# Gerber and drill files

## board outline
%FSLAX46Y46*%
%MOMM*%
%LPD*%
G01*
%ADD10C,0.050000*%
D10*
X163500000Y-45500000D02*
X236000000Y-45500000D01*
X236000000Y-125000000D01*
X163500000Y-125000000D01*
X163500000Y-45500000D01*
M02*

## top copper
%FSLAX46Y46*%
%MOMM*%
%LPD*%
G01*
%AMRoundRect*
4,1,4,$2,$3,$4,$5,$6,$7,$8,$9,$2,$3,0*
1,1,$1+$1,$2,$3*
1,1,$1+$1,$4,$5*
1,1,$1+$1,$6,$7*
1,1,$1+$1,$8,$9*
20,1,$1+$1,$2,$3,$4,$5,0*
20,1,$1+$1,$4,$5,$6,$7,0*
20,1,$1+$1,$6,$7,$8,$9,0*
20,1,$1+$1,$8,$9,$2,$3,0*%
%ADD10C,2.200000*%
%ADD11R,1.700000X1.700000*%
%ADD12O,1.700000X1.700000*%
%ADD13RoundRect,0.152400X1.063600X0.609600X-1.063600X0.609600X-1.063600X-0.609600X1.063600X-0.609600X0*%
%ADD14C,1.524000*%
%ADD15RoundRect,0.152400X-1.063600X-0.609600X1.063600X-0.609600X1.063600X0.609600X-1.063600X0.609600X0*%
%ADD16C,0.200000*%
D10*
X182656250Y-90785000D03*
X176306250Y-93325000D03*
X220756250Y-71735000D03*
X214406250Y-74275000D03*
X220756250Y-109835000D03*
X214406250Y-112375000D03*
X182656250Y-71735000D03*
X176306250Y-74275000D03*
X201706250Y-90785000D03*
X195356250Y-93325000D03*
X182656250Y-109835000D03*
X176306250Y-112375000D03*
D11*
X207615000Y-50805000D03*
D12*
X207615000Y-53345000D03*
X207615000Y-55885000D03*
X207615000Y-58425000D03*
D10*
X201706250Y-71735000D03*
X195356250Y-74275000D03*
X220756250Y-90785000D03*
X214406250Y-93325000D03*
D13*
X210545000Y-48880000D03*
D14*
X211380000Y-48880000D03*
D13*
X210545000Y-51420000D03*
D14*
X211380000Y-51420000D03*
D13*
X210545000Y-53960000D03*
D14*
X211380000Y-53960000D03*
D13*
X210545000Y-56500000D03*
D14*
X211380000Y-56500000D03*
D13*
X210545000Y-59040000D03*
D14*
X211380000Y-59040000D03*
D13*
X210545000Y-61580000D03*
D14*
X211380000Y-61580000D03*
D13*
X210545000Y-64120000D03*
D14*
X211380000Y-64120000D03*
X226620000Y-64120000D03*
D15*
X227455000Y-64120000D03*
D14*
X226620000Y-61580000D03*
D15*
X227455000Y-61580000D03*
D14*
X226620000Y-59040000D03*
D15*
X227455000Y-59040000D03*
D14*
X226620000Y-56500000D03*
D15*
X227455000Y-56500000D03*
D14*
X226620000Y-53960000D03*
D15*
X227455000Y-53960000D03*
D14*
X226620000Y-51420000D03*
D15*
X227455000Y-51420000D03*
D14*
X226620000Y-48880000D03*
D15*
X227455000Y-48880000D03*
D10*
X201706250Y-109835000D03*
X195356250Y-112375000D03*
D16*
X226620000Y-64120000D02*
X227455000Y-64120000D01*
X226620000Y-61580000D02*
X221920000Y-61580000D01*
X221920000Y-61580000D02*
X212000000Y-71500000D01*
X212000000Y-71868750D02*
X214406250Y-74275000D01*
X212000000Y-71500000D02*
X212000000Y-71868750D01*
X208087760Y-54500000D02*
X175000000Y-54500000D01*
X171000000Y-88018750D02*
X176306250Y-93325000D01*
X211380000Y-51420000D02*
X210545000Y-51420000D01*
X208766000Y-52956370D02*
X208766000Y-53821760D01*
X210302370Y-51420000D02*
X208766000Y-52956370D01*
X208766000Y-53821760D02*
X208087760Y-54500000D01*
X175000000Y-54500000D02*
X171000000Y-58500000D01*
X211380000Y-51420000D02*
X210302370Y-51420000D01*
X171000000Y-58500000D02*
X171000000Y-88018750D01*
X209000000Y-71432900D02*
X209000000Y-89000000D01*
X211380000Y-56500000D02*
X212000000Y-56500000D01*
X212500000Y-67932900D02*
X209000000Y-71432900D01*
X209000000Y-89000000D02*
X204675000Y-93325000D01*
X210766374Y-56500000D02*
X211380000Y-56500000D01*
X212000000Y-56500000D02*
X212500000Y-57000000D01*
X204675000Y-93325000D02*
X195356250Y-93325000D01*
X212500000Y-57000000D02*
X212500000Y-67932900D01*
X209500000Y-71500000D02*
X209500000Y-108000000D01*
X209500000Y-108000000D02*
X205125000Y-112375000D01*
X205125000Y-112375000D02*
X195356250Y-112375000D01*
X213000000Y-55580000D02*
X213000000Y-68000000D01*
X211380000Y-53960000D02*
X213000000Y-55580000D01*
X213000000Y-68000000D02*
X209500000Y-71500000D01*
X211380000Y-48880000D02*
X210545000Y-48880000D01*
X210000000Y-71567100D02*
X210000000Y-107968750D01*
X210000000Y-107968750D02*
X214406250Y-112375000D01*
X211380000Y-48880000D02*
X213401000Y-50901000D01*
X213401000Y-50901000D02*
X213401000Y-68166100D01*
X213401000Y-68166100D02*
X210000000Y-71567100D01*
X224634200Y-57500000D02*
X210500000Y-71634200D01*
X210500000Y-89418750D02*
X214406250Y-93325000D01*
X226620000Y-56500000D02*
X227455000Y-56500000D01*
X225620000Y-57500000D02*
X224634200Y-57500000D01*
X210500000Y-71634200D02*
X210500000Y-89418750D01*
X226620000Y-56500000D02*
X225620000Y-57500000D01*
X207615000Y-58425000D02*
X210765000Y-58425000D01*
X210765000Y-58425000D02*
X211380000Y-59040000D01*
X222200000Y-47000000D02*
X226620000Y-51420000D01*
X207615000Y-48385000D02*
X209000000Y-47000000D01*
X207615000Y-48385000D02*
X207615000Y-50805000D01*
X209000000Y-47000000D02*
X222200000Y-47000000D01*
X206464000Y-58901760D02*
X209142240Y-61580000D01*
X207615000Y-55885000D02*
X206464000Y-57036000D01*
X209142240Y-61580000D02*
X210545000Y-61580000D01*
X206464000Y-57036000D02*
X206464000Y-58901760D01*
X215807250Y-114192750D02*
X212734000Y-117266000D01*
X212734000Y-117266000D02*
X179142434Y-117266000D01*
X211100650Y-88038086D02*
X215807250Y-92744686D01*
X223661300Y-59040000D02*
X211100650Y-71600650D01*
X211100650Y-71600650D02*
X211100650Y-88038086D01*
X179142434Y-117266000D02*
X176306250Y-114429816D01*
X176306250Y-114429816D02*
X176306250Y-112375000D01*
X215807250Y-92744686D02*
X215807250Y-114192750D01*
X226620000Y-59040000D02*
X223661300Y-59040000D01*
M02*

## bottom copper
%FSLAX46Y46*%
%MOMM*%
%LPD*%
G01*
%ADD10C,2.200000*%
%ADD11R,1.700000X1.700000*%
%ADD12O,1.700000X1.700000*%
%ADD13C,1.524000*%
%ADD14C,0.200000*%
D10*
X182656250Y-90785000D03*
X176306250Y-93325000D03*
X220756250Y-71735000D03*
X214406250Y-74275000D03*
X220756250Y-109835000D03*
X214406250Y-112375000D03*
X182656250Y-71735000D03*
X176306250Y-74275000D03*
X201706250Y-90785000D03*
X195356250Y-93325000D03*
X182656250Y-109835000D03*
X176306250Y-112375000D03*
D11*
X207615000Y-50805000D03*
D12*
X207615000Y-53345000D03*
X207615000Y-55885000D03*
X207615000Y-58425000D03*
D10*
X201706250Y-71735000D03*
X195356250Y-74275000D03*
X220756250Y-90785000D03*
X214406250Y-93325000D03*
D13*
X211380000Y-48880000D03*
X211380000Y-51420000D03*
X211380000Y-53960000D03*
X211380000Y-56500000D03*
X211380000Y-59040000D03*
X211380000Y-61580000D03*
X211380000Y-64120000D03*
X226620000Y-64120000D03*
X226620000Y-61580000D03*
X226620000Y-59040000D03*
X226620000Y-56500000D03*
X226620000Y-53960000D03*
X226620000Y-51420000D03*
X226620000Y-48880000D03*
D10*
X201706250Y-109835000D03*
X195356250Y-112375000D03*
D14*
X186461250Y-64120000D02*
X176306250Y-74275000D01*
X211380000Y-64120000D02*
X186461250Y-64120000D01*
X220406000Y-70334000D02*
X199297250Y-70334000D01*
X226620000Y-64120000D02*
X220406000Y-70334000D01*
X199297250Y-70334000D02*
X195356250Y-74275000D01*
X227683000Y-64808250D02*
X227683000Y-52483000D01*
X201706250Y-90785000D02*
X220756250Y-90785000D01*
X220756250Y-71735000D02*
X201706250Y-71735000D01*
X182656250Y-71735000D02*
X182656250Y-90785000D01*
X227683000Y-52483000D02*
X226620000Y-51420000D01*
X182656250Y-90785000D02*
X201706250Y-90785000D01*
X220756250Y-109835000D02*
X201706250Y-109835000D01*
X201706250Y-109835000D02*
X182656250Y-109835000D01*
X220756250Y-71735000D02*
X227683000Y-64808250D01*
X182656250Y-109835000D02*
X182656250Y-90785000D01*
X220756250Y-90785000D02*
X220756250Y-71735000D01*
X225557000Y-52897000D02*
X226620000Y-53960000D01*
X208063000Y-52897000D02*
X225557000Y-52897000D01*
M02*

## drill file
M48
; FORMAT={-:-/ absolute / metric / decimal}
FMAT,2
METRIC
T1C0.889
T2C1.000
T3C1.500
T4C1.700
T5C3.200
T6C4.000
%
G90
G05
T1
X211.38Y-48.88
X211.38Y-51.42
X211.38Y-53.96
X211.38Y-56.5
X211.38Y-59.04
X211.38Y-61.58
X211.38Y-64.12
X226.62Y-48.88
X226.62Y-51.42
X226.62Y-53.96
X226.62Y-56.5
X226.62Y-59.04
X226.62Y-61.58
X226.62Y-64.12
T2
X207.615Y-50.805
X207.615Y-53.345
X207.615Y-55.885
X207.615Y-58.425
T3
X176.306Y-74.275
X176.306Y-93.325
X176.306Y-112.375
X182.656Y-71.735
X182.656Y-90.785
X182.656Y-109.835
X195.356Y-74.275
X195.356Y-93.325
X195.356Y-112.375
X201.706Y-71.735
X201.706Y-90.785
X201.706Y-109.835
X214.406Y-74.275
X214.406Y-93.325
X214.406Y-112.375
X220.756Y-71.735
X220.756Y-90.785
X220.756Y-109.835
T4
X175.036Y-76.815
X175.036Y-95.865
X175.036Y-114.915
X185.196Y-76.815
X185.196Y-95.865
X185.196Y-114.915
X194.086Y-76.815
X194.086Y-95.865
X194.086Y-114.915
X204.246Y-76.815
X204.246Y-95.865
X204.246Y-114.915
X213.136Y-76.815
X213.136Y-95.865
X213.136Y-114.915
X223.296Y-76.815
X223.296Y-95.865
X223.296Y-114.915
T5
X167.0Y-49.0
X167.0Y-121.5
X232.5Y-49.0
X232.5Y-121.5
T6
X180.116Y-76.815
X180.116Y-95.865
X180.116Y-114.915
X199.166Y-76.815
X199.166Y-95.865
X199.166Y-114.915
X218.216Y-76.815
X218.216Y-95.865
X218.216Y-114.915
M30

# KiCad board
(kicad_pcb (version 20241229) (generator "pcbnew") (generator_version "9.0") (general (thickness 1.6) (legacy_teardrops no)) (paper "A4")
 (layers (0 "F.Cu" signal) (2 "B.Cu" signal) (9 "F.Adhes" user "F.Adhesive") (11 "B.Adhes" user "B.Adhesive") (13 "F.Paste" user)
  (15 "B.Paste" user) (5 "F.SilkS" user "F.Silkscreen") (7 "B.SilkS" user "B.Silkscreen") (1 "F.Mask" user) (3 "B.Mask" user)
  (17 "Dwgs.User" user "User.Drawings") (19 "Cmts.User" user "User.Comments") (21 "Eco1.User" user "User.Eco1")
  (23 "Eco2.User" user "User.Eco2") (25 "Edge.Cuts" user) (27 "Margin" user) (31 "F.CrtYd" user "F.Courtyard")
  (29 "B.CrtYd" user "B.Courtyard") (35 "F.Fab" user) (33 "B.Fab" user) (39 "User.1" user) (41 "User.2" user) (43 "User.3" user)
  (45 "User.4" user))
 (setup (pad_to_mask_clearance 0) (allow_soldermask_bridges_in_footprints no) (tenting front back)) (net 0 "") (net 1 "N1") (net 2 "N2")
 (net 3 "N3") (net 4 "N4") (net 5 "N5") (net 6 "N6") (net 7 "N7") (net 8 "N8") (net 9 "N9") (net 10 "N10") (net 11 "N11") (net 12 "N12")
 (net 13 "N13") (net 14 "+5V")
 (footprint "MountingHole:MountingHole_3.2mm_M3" (layer "F.Cu") (at 232.5 49)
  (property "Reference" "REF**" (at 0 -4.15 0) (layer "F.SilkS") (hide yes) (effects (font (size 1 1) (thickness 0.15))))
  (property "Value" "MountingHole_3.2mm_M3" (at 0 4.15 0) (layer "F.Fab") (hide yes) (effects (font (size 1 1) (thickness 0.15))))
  (pad "" np_thru_hole circle (at 0 0) (size 3.2 3.2) (drill 3.2) (layers "*.Cu" "*.Mask")))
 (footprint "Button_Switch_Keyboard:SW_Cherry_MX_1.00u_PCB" (layer "F.Cu") (at 182.65625 90.785)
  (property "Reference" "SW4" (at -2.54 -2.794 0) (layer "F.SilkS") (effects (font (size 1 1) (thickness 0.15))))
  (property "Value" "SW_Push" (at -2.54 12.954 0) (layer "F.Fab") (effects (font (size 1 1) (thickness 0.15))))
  (pad "" np_thru_hole circle (at -7.62 5.08) (size 1.7 1.7) (drill 1.7) (layers "*.Cu" "*.Mask"))
  (pad "" np_thru_hole circle (at -2.54 5.08) (size 4 4) (drill 4) (layers "*.Cu" "*.Mask"))
  (pad "" np_thru_hole circle (at 2.54 5.08) (size 1.7 1.7) (drill 1.7) (layers "*.Cu" "*.Mask"))
  (pad "1" thru_hole circle (at 0 0) (size 2.2 2.2) (drill 1.5) (layers "*.Cu" "*.Mask") (remove_unused_layers no) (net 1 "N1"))
  (pad "2" thru_hole circle (at -6.35 2.54) (size 2.2 2.2) (drill 1.5) (layers "*.Cu" "*.Mask") (remove_unused_layers no) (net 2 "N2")))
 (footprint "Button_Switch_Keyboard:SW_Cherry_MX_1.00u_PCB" (layer "F.Cu") (at 220.75625 71.735)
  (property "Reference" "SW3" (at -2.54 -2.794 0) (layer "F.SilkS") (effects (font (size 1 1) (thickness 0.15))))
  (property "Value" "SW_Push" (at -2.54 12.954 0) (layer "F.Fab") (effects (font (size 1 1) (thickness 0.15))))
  (pad "" np_thru_hole circle (at -7.62 5.08) (size 1.7 1.7) (drill 1.7) (layers "*.Cu" "*.Mask"))
  (pad "" np_thru_hole circle (at -2.54 5.08) (size 4 4) (drill 4) (layers "*.Cu" "*.Mask"))
  (pad "" np_thru_hole circle (at 2.54 5.08) (size 1.7 1.7) (drill 1.7) (layers "*.Cu" "*.Mask"))
  (pad "1" thru_hole circle (at 0 0) (size 2.2 2.2) (drill 1.5) (layers "*.Cu" "*.Mask") (remove_unused_layers no) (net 1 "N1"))
  (pad "2" thru_hole circle (at -6.35 2.54) (size 2.2 2.2) (drill 1.5) (layers "*.Cu" "*.Mask") (remove_unused_layers no) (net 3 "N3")))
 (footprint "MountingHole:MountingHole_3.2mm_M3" (layer "F.Cu") (at 167 121.5)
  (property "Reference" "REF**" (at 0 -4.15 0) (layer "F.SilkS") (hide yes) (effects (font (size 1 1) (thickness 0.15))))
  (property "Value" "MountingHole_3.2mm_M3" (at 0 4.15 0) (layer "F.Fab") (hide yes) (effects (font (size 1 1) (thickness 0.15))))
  (pad "" np_thru_hole circle (at 0 0) (size 3.2 3.2) (drill 3.2) (layers "*.Cu" "*.Mask")))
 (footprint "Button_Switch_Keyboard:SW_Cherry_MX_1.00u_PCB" (layer "F.Cu") (at 220.75625 109.835)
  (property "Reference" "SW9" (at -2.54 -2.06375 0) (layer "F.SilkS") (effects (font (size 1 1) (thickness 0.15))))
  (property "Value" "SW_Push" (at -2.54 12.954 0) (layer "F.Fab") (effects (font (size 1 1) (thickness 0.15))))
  (pad "" np_thru_hole circle (at -7.62 5.08) (size 1.7 1.7) (drill 1.7) (layers "*.Cu" "*.Mask"))
  (pad "" np_thru_hole circle (at -2.54 5.08) (size 4 4) (drill 4) (layers "*.Cu" "*.Mask"))
  (pad "" np_thru_hole circle (at 2.54 5.08) (size 1.7 1.7) (drill 1.7) (layers "*.Cu" "*.Mask"))
  (pad "1" thru_hole circle (at 0 0) (size 2.2 2.2) (drill 1.5) (layers "*.Cu" "*.Mask") (remove_unused_layers no) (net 1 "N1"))
  (pad "2" thru_hole circle (at -6.35 2.54) (size 2.2 2.2) (drill 1.5) (layers "*.Cu" "*.Mask") (remove_unused_layers no) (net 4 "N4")))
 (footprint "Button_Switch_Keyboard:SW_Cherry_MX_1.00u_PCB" (layer "F.Cu") (at 182.65625 71.735)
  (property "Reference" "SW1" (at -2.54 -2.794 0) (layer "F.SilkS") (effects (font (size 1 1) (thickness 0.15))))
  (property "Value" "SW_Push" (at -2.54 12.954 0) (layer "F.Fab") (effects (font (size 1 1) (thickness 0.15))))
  (pad "" np_thru_hole circle (at -7.62 5.08) (size 1.7 1.7) (drill 1.7) (layers "*.Cu" "*.Mask"))
  (pad "" np_thru_hole circle (at -2.54 5.08) (size 4 4) (drill 4) (layers "*.Cu" "*.Mask"))
  (pad "" np_thru_hole circle (at 2.54 5.08) (size 1.7 1.7) (drill 1.7) (layers "*.Cu" "*.Mask"))
  (pad "1" thru_hole circle (at 0 0) (size 2.2 2.2) (drill 1.5) (layers "*.Cu" "*.Mask") (remove_unused_layers no) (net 1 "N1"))
  (pad "2" thru_hole circle (at -6.35 2.54) (size 2.2 2.2) (drill 1.5) (layers "*.Cu" "*.Mask") (remove_unused_layers no) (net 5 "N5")))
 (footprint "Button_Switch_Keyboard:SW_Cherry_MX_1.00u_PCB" (layer "F.Cu") (at 201.70625 90.785)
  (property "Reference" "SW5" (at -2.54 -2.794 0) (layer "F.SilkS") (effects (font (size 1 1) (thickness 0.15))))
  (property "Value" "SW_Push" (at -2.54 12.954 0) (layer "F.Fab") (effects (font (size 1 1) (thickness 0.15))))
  (pad "" np_thru_hole circle (at -7.62 5.08) (size 1.7 1.7) (drill 1.7) (layers "*.Cu" "*.Mask"))
  (pad "" np_thru_hole circle (at -2.54 5.08) (size 4 4) (drill 4) (layers "*.Cu" "*.Mask"))
  (pad "" np_thru_hole circle (at 2.54 5.08) (size 1.7 1.7) (drill 1.7) (layers "*.Cu" "*.Mask"))
  (pad "1" thru_hole circle (at 0 0) (size 2.2 2.2) (drill 1.5) (layers "*.Cu" "*.Mask") (remove_unused_layers no) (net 1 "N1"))
  (pad "2" thru_hole circle (at -6.35 2.54) (size 2.2 2.2) (drill 1.5) (layers "*.Cu" "*.Mask") (remove_unused_layers no) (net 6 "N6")))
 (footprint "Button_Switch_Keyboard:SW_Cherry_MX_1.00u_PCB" (layer "F.Cu") (at 182.65625 109.835)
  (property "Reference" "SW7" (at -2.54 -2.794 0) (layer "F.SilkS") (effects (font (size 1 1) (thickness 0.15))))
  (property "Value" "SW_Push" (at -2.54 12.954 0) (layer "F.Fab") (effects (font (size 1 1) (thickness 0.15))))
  (pad "" np_thru_hole circle (at -7.62 5.08) (size 1.7 1.7) (drill 1.7) (layers "*.Cu" "*.Mask"))
  (pad "" np_thru_hole circle (at -2.54 5.08) (size 4 4) (drill 4) (layers "*.Cu" "*.Mask"))
  (pad "" np_thru_hole circle (at 2.54 5.08) (size 1.7 1.7) (drill 1.7) (layers "*.Cu" "*.Mask"))
  (pad "1" thru_hole circle (at 0 0) (size 2.2 2.2) (drill 1.5) (layers "*.Cu" "*.Mask") (remove_unused_layers no) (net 1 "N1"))
  (pad "2" thru_hole circle (at -6.35 2.54) (size 2.2 2.2) (drill 1.5) (layers "*.Cu" "*.Mask") (remove_unused_layers no) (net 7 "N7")))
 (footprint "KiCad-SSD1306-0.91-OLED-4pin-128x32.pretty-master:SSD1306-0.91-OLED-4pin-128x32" (layer "F.Cu") (at 171.115 48.615)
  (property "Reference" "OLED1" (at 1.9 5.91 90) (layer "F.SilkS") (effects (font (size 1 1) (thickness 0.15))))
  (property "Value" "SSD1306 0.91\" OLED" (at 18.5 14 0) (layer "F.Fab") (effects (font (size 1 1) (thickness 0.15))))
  (pad "1" thru_hole rect (at 36.5 2.19) (size 1.7 1.7) (drill 1) (layers "*.Cu" "*.Mask") (remove_unused_layers no) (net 1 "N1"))
  (pad "2" thru_hole oval (at 36.5 4.73) (size 1.7 1.7) (drill 1) (layers "*.Cu" "*.Mask") (remove_unused_layers no) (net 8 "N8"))
  (pad "3" thru_hole oval (at 36.5 7.27) (size 1.7 1.7) (drill 1) (layers "*.Cu" "*.Mask") (remove_unused_layers no) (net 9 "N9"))
  (pad "4" thru_hole oval (at 36.5 9.81) (size 1.7 1.7) (drill 1) (layers "*.Cu" "*.Mask") (remove_unused_layers no) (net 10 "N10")))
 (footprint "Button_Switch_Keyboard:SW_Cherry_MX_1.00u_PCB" (layer "F.Cu") (at 201.70625 71.735)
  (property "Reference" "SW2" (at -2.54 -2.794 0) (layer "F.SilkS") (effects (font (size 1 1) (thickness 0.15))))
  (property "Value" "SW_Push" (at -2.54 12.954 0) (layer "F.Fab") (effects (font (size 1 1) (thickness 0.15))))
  (pad "" np_thru_hole circle (at -7.62 5.08) (size 1.7 1.7) (drill 1.7) (layers "*.Cu" "*.Mask"))
  (pad "" np_thru_hole circle (at -2.54 5.08) (size 4 4) (drill 4) (layers "*.Cu" "*.Mask"))
  (pad "" np_thru_hole circle (at 2.54 5.08) (size 1.7 1.7) (drill 1.7) (layers "*.Cu" "*.Mask"))
  (pad "1" thru_hole circle (at 0 0) (size 2.2 2.2) (drill 1.5) (layers "*.Cu" "*.Mask") (remove_unused_layers no) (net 1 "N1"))
  (pad "2" thru_hole circle (at -6.35 2.54) (size 2.2 2.2) (drill 1.5) (layers "*.Cu" "*.Mask") (remove_unused_layers no) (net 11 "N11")))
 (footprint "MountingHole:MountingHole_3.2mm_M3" (layer "F.Cu") (at 167 49)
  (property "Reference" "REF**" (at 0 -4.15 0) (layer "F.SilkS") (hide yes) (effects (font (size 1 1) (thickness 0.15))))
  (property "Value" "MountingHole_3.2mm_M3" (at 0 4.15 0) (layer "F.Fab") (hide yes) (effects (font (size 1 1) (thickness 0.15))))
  (pad "" np_thru_hole circle (at 0 0) (size 3.2 3.2) (drill 3.2) (layers "*.Cu" "*.Mask")))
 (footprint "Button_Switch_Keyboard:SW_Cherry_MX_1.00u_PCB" (layer "F.Cu") (at 220.75625 90.785)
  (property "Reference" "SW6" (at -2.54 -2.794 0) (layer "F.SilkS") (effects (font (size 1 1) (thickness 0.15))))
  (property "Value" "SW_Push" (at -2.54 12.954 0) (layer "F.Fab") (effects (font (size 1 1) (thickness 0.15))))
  (pad "" np_thru_hole circle (at -7.62 5.08) (size 1.7 1.7) (drill 1.7) (layers "*.Cu" "*.Mask"))
  (pad "" np_thru_hole circle (at -2.54 5.08) (size 4 4) (drill 4) (layers "*.Cu" "*.Mask"))
  (pad "" np_thru_hole circle (at 2.54 5.08) (size 1.7 1.7) (drill 1.7) (layers "*.Cu" "*.Mask"))
  (pad "1" thru_hole circle (at 0 0) (size 2.2 2.2) (drill 1.5) (layers "*.Cu" "*.Mask") (remove_unused_layers no) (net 1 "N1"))
  (pad "2" thru_hole circle (at -6.35 2.54) (size 2.2 2.2) (drill 1.5) (layers "*.Cu" "*.Mask") (remove_unused_layers no) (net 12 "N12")))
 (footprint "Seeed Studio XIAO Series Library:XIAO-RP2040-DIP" (layer "F.Cu") (at 219 56.5)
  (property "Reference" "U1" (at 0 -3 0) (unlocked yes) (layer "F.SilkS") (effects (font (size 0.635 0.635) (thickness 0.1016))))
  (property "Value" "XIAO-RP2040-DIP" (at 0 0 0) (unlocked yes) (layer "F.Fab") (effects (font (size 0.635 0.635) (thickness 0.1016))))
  (pad "1" smd roundrect (at -8.455 -7.62 180) (size 2.432 1.524) (layers "F.Cu" "F.Mask") (roundrect_rratio 0.1) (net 4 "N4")
   (thermal_bridge_angle 45))
  (pad "1" thru_hole circle (at -7.62 -7.62 180) (size 1.524 1.524) (drill 0.889) (layers "*.Cu" "*.Mask") (remove_unused_layers no)
   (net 4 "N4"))
  (pad "2" smd roundrect (at -8.455 -5.08 180) (size 2.432 1.524) (layers "F.Cu" "F.Mask") (roundrect_rratio 0.1) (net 2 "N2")
   (thermal_bridge_angle 45))
  (pad "2" thru_hole circle (at -7.62 -5.08 180) (size 1.524 1.524) (drill 0.889) (layers "*.Cu" "*.Mask") (remove_unused_layers no)
   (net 2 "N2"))
  (pad "3" smd roundrect (at -8.455 -2.54 180) (size 2.432 1.524) (layers "F.Cu" "F.Mask") (roundrect_rratio 0.1) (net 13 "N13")
   (thermal_bridge_angle 45))
  (pad "3" thru_hole circle (at -7.62 -2.54 180) (size 1.524 1.524) (drill 0.889) (layers "*.Cu" "*.Mask") (remove_unused_layers no)
   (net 13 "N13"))
  (pad "4" smd roundrect (at -8.455 0 180) (size 2.432 1.524) (layers "F.Cu" "F.Mask") (roundrect_rratio 0.1) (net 6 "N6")
   (thermal_bridge_angle 45))
  (pad "4" thru_hole circle (at -7.62 0 180) (size 1.524 1.524) (drill 0.889) (layers "*.Cu" "*.Mask") (remove_unused_layers no)
   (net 6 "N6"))
  (pad "5" smd roundrect (at -8.455 2.54 180) (size 2.432 1.524) (layers "F.Cu" "F.Mask") (roundrect_rratio 0.1) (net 10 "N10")
   (thermal_bridge_angle 45))
  (pad "5" thru_hole circle (at -7.62 2.54 180) (size 1.524 1.524) (drill 0.889) (layers "*.Cu" "*.Mask") (remove_unused_layers no)
   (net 10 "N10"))
  (pad "6" smd roundrect (at -8.455 5.08 180) (size 2.432 1.524) (layers "F.Cu" "F.Mask") (roundrect_rratio 0.1) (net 9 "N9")
   (thermal_bridge_angle 45))
  (pad "6" thru_hole circle (at -7.62 5.08 180) (size 1.524 1.524) (drill 0.889) (layers "*.Cu" "*.Mask") (remove_unused_layers no)
   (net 9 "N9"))
  (pad "7" smd roundrect (at -8.455 7.62 180) (size 2.432 1.524) (layers "F.Cu" "F.Mask") (roundrect_rratio 0.1) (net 5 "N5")
   (thermal_bridge_angle 45))
  (pad "7" thru_hole circle (at -7.62 7.62 180) (size 1.524 1.524) (drill 0.889) (layers "*.Cu" "*.Mask") (remove_unused_layers no)
   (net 5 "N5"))
  (pad "8" thru_hole circle (at 7.62 7.62) (size 1.524 1.524) (drill 0.889) (layers "*.Cu" "*.Mask") (remove_unused_layers no)
   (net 11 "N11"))
  (pad "8" smd roundrect (at 8.455 7.62) (size 2.432 1.524) (layers "F.Cu" "F.Mask") (roundrect_rratio 0.1) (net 11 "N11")
   (thermal_bridge_angle 45))
  (pad "9" thru_hole circle (at 7.62 5.08) (size 1.524 1.524) (drill 0.889) (layers "*.Cu" "*.Mask") (remove_unused_layers no) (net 3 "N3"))
  (pad "9" smd roundrect (at 8.455 5.08) (size 2.432 1.524) (layers "F.Cu" "F.Mask") (roundrect_rratio 0.1) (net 3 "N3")
   (thermal_bridge_angle 45))
  (pad "10" thru_hole circle (at 7.62 2.54) (size 1.524 1.524) (drill 0.889) (layers "*.Cu" "*.Mask") (remove_unused_layers no) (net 7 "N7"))
  (pad "10" smd roundrect (at 8.455 2.54) (size 2.432 1.524) (layers "F.Cu" "F.Mask") (roundrect_rratio 0.1) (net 7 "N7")
   (thermal_bridge_angle 45))
  (pad "11" thru_hole circle (at 7.62 0) (size 1.524 1.524) (drill 0.889) (layers "*.Cu" "*.Mask") (remove_unused_layers no) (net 12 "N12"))
  (pad "11" smd roundrect (at 8.455 0) (size 2.432 1.524) (layers "F.Cu" "F.Mask") (roundrect_rratio 0.1) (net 12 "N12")
   (thermal_bridge_angle 45))
  (pad "12" thru_hole circle (at 7.62 -2.54) (size 1.524 1.524) (drill 0.889) (layers "*.Cu" "*.Mask") (remove_unused_layers no)
   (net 8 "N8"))
  (pad "12" smd roundrect (at 8.455 -2.54) (size 2.432 1.524) (layers "F.Cu" "F.Mask") (roundrect_rratio 0.1) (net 8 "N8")
   (thermal_bridge_angle 45))
  (pad "13" thru_hole circle (at 7.62 -5.08) (size 1.524 1.524) (drill 0.889) (layers "*.Cu" "*.Mask") (remove_unused_layers no)
   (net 1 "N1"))
  (pad "13" smd roundrect (at 8.455 -5.08) (size 2.432 1.524) (layers "F.Cu" "F.Mask") (roundrect_rratio 0.1) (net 1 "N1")
   (thermal_bridge_angle 45))
  (pad "14" thru_hole circle (at 7.62 -7.62) (size 1.524 1.524) (drill 0.889) (layers "*.Cu" "*.Mask") (remove_unused_layers no)
   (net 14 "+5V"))
  (pad "14" smd roundrect (at 8.455 -7.62) (size 2.432 1.524) (layers "F.Cu" "F.Mask") (roundrect_rratio 0.1) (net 14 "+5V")
   (thermal_bridge_angle 45)))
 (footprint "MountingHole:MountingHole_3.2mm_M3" (layer "F.Cu") (at 232.5 121.5)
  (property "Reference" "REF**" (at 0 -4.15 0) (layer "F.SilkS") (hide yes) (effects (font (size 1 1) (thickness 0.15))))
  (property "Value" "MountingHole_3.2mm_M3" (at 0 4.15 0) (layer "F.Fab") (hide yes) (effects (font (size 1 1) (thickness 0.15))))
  (pad "" np_thru_hole circle (at 0 0) (size 3.2 3.2) (drill 3.2) (layers "*.Cu" "*.Mask")))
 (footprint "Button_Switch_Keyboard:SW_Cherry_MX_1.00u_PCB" (layer "F.Cu") (at 201.70625 109.835)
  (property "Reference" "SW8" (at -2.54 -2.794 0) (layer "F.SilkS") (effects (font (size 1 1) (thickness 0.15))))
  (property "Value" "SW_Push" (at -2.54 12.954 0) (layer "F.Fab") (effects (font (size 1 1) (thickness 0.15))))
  (pad "" np_thru_hole circle (at -7.62 5.08) (size 1.7 1.7) (drill 1.7) (layers "*.Cu" "*.Mask"))
  (pad "" np_thru_hole circle (at -2.54 5.08) (size 4 4) (drill 4) (layers "*.Cu" "*.Mask"))
  (pad "" np_thru_hole circle (at 2.54 5.08) (size 1.7 1.7) (drill 1.7) (layers "*.Cu" "*.Mask"))
  (pad "1" thru_hole circle (at 0 0) (size 2.2 2.2) (drill 1.5) (layers "*.Cu" "*.Mask") (remove_unused_layers no) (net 1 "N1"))
  (pad "2" thru_hole circle (at -6.35 2.54) (size 2.2 2.2) (drill 1.5) (layers "*.Cu" "*.Mask") (remove_unused_layers no) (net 13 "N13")))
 (gr_rect (start 163.5 45.5) (end 236 125) (stroke (width 0.05) (type default)) (fill no) (layer "Edge.Cuts"))
 (segment (start 186.46125 64.12) (end 176.30625 74.275) (width 0.2) (layer "B.Cu") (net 5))
 (segment (start 211.38 64.12) (end 186.46125 64.12) (width 0.2) (layer "B.Cu") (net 5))
 (segment (start 226.62 64.12) (end 227.455 64.12) (width 0.2) (layer "F.Cu") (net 11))
 (segment (start 220.406 70.334) (end 199.29725 70.334) (width 0.2) (layer "B.Cu") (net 11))
 (segment (start 226.62 64.12) (end 220.406 70.334) (width 0.2) (layer "B.Cu") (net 11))
 (segment (start 199.29725 70.334) (end 195.35625 74.275) (width 0.2) (layer "B.Cu") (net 11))
 (segment (start 226.62 61.58) (end 221.92 61.58) (width 0.2) (layer "F.Cu") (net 3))
 (segment (start 221.92 61.58) (end 212 71.5) (width 0.2) (layer "F.Cu") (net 3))
 (segment (start 212 71.86875) (end 214.40625 74.275) (width 0.2) (layer "F.Cu") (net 3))
 (segment (start 212 71.5) (end 212 71.86875) (width 0.2) (layer "F.Cu") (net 3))
 (segment (start 208.08776 54.5) (end 175 54.5) (width 0.2) (layer "F.Cu") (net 2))
 (segment (start 171 88.01875) (end 176.30625 93.325) (width 0.2) (layer "F.Cu") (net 2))
 (segment (start 211.38 51.42) (end 210.545 51.42) (width 0.2) (layer "F.Cu") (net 2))
 (segment (start 208.766 52.95637) (end 208.766 53.82176) (width 0.2) (layer "F.Cu") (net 2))
 (segment (start 210.30237 51.42) (end 208.766 52.95637) (width 0.2) (layer "F.Cu") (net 2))
 (segment (start 208.766 53.82176) (end 208.08776 54.5) (width 0.2) (layer "F.Cu") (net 2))
 (segment (start 175 54.5) (end 171 58.5) (width 0.2) (layer "F.Cu") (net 2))
 (segment (start 211.38 51.42) (end 210.30237 51.42) (width 0.2) (layer "F.Cu") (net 2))
 (segment (start 171 58.5) (end 171 88.01875) (width 0.2) (layer "F.Cu") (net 2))
 (segment (start 209 71.4329) (end 209 89) (width 0.2) (layer "F.Cu") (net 6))
 (segment (start 211.38 56.5) (end 212 56.5) (width 0.2) (layer "F.Cu") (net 6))
 (segment (start 212.5 67.9329) (end 209 71.4329) (width 0.2) (layer "F.Cu") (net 6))
 (segment (start 209 89) (end 204.675 93.325) (width 0.2) (layer "F.Cu") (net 6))
 (segment (start 210.766374 56.5) (end 211.38 56.5) (width 0.2) (layer "F.Cu") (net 6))
 (segment (start 212 56.5) (end 212.5 57) (width 0.2) (layer "F.Cu") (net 6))
 (segment (start 204.675 93.325) (end 195.35625 93.325) (width 0.2) (layer "F.Cu") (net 6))
 (segment (start 212.5 57) (end 212.5 67.9329) (width 0.2) (layer "F.Cu") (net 6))
 (segment (start 209.5 71.5) (end 209.5 108) (width 0.2) (layer "F.Cu") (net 13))
 (segment (start 209.5 108) (end 205.125 112.375) (width 0.2) (layer "F.Cu") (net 13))
 (segment (start 205.125 112.375) (end 195.35625 112.375) (width 0.2) (layer "F.Cu") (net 13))
 (segment (start 213 55.58) (end 213 68) (width 0.2) (layer "F.Cu") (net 13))
 (segment (start 211.38 53.96) (end 213 55.58) (width 0.2) (layer "F.Cu") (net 13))
 (segment (start 213 68) (end 209.5 71.5) (width 0.2) (layer "F.Cu") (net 13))
 (segment (start 211.38 48.88) (end 210.545 48.88) (width 0.2) (layer "F.Cu") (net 4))
 (segment (start 210 71.5671) (end 210 107.96875) (width 0.2) (layer "F.Cu") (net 4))
 (segment (start 210 107.96875) (end 214.40625 112.375) (width 0.2) (layer "F.Cu") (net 4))
 (segment (start 211.38 48.88) (end 213.401 50.901) (width 0.2) (layer "F.Cu") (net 4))
 (segment (start 213.401 50.901) (end 213.401 68.1661) (width 0.2) (layer "F.Cu") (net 4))
 (segment (start 213.401 68.1661) (end 210 71.5671) (width 0.2) (layer "F.Cu") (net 4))
 (segment (start 224.6342 57.5) (end 210.5 71.6342) (width 0.2) (layer "F.Cu") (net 12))
 (segment (start 210.5 89.41875) (end 214.40625 93.325) (width 0.2) (layer "F.Cu") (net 12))
 (segment (start 226.62 56.5) (end 227.455 56.5) (width 0.2) (layer "F.Cu") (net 12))
 (segment (start 225.62 57.5) (end 224.6342 57.5) (width 0.2) (layer "F.Cu") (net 12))
 (segment (start 210.5 71.6342) (end 210.5 89.41875) (width 0.2) (layer "F.Cu") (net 12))
 (segment (start 226.62 56.5) (end 225.62 57.5) (width 0.2) (layer "F.Cu") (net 12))
 (segment (start 207.615 58.425) (end 210.765 58.425) (width 0.2) (layer "F.Cu") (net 10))
 (segment (start 210.765 58.425) (end 211.38 59.04) (width 0.2) (layer "F.Cu") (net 10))
 (segment (start 222.2 47) (end 226.62 51.42) (width 0.2) (layer "F.Cu") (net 1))
 (segment (start 207.615 48.385) (end 209 47) (width 0.2) (layer "F.Cu") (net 1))
 (segment (start 207.615 48.385) (end 207.615 50.805) (width 0.2) (layer "F.Cu") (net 1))
 (segment (start 209 47) (end 222.2 47) (width 0.2) (layer "F.Cu") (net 1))
 (segment (start 227.683 64.80825) (end 227.683 52.483) (width 0.2) (layer "B.Cu") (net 1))
 (segment (start 201.70625 90.785) (end 220.75625 90.785) (width 0.2) (layer "B.Cu") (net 1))
 (segment (start 220.75625 71.735) (end 201.70625 71.735) (width 0.2) (layer "B.Cu") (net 1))
 (segment (start 182.65625 71.735) (end 182.65625 90.785) (width 0.2) (layer "B.Cu") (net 1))
 (segment (start 227.683 52.483) (end 226.62 51.42) (width 0.2) (layer "B.Cu") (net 1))
 (segment (start 182.65625 90.785) (end 201.70625 90.785) (width 0.2) (layer "B.Cu") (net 1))
 (segment (start 220.75625 109.835) (end 201.70625 109.835) (width 0.2) (layer "B.Cu") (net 1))
 (segment (start 201.70625 109.835) (end 182.65625 109.835) (width 0.2) (layer "B.Cu") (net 1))
 (segment (start 220.75625 71.735) (end 227.683 64.80825) (width 0.2) (layer "B.Cu") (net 1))
 (segment (start 182.65625 109.835) (end 182.65625 90.785) (width 0.2) (layer "B.Cu") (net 1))
 (segment (start 220.75625 90.785) (end 220.75625 71.735) (width 0.2) (layer "B.Cu") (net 1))
 (segment (start 225.557 52.897) (end 226.62 53.96) (width 0.2) (layer "B.Cu") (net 8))
 (segment (start 208.063 52.897) (end 225.557 52.897) (width 0.2) (layer "B.Cu") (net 8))
 (segment (start 206.464 58.90176) (end 209.14224 61.58) (width 0.2) (layer "F.Cu") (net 9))
 (segment (start 207.615 55.885) (end 206.464 57.036) (width 0.2) (layer "F.Cu") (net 9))
 (segment (start 209.14224 61.58) (end 210.545 61.58) (width 0.2) (layer "F.Cu") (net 9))
 (segment (start 206.464 57.036) (end 206.464 58.90176) (width 0.2) (layer "F.Cu") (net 9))
 (segment (start 215.80725 114.19275) (end 212.734 117.266) (width 0.2) (layer "F.Cu") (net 7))
 (segment (start 212.734 117.266) (end 179.142434 117.266) (width 0.2) (layer "F.Cu") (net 7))
 (segment (start 211.10065 88.038086) (end 215.80725 92.744686) (width 0.2) (layer "F.Cu") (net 7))
 (segment (start 223.6613 59.04) (end 211.10065 71.60065) (width 0.2) (layer "F.Cu") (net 7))
 (segment (start 211.10065 71.60065) (end 211.10065 88.038086) (width 0.2) (layer "F.Cu") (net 7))
 (segment (start 179.142434 117.266) (end 176.30625 114.429816) (width 0.2) (layer "F.Cu") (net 7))
 (segment (start 176.30625 114.429816) (end 176.30625 112.375) (width 0.2) (layer "F.Cu") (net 7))
 (segment (start 215.80725 92.744686) (end 215.80725 114.19275) (width 0.2) (layer "F.Cu") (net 7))
 (segment (start 226.62 59.04) (end 223.6613 59.04) (width 0.2) (layer "F.Cu") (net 7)))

